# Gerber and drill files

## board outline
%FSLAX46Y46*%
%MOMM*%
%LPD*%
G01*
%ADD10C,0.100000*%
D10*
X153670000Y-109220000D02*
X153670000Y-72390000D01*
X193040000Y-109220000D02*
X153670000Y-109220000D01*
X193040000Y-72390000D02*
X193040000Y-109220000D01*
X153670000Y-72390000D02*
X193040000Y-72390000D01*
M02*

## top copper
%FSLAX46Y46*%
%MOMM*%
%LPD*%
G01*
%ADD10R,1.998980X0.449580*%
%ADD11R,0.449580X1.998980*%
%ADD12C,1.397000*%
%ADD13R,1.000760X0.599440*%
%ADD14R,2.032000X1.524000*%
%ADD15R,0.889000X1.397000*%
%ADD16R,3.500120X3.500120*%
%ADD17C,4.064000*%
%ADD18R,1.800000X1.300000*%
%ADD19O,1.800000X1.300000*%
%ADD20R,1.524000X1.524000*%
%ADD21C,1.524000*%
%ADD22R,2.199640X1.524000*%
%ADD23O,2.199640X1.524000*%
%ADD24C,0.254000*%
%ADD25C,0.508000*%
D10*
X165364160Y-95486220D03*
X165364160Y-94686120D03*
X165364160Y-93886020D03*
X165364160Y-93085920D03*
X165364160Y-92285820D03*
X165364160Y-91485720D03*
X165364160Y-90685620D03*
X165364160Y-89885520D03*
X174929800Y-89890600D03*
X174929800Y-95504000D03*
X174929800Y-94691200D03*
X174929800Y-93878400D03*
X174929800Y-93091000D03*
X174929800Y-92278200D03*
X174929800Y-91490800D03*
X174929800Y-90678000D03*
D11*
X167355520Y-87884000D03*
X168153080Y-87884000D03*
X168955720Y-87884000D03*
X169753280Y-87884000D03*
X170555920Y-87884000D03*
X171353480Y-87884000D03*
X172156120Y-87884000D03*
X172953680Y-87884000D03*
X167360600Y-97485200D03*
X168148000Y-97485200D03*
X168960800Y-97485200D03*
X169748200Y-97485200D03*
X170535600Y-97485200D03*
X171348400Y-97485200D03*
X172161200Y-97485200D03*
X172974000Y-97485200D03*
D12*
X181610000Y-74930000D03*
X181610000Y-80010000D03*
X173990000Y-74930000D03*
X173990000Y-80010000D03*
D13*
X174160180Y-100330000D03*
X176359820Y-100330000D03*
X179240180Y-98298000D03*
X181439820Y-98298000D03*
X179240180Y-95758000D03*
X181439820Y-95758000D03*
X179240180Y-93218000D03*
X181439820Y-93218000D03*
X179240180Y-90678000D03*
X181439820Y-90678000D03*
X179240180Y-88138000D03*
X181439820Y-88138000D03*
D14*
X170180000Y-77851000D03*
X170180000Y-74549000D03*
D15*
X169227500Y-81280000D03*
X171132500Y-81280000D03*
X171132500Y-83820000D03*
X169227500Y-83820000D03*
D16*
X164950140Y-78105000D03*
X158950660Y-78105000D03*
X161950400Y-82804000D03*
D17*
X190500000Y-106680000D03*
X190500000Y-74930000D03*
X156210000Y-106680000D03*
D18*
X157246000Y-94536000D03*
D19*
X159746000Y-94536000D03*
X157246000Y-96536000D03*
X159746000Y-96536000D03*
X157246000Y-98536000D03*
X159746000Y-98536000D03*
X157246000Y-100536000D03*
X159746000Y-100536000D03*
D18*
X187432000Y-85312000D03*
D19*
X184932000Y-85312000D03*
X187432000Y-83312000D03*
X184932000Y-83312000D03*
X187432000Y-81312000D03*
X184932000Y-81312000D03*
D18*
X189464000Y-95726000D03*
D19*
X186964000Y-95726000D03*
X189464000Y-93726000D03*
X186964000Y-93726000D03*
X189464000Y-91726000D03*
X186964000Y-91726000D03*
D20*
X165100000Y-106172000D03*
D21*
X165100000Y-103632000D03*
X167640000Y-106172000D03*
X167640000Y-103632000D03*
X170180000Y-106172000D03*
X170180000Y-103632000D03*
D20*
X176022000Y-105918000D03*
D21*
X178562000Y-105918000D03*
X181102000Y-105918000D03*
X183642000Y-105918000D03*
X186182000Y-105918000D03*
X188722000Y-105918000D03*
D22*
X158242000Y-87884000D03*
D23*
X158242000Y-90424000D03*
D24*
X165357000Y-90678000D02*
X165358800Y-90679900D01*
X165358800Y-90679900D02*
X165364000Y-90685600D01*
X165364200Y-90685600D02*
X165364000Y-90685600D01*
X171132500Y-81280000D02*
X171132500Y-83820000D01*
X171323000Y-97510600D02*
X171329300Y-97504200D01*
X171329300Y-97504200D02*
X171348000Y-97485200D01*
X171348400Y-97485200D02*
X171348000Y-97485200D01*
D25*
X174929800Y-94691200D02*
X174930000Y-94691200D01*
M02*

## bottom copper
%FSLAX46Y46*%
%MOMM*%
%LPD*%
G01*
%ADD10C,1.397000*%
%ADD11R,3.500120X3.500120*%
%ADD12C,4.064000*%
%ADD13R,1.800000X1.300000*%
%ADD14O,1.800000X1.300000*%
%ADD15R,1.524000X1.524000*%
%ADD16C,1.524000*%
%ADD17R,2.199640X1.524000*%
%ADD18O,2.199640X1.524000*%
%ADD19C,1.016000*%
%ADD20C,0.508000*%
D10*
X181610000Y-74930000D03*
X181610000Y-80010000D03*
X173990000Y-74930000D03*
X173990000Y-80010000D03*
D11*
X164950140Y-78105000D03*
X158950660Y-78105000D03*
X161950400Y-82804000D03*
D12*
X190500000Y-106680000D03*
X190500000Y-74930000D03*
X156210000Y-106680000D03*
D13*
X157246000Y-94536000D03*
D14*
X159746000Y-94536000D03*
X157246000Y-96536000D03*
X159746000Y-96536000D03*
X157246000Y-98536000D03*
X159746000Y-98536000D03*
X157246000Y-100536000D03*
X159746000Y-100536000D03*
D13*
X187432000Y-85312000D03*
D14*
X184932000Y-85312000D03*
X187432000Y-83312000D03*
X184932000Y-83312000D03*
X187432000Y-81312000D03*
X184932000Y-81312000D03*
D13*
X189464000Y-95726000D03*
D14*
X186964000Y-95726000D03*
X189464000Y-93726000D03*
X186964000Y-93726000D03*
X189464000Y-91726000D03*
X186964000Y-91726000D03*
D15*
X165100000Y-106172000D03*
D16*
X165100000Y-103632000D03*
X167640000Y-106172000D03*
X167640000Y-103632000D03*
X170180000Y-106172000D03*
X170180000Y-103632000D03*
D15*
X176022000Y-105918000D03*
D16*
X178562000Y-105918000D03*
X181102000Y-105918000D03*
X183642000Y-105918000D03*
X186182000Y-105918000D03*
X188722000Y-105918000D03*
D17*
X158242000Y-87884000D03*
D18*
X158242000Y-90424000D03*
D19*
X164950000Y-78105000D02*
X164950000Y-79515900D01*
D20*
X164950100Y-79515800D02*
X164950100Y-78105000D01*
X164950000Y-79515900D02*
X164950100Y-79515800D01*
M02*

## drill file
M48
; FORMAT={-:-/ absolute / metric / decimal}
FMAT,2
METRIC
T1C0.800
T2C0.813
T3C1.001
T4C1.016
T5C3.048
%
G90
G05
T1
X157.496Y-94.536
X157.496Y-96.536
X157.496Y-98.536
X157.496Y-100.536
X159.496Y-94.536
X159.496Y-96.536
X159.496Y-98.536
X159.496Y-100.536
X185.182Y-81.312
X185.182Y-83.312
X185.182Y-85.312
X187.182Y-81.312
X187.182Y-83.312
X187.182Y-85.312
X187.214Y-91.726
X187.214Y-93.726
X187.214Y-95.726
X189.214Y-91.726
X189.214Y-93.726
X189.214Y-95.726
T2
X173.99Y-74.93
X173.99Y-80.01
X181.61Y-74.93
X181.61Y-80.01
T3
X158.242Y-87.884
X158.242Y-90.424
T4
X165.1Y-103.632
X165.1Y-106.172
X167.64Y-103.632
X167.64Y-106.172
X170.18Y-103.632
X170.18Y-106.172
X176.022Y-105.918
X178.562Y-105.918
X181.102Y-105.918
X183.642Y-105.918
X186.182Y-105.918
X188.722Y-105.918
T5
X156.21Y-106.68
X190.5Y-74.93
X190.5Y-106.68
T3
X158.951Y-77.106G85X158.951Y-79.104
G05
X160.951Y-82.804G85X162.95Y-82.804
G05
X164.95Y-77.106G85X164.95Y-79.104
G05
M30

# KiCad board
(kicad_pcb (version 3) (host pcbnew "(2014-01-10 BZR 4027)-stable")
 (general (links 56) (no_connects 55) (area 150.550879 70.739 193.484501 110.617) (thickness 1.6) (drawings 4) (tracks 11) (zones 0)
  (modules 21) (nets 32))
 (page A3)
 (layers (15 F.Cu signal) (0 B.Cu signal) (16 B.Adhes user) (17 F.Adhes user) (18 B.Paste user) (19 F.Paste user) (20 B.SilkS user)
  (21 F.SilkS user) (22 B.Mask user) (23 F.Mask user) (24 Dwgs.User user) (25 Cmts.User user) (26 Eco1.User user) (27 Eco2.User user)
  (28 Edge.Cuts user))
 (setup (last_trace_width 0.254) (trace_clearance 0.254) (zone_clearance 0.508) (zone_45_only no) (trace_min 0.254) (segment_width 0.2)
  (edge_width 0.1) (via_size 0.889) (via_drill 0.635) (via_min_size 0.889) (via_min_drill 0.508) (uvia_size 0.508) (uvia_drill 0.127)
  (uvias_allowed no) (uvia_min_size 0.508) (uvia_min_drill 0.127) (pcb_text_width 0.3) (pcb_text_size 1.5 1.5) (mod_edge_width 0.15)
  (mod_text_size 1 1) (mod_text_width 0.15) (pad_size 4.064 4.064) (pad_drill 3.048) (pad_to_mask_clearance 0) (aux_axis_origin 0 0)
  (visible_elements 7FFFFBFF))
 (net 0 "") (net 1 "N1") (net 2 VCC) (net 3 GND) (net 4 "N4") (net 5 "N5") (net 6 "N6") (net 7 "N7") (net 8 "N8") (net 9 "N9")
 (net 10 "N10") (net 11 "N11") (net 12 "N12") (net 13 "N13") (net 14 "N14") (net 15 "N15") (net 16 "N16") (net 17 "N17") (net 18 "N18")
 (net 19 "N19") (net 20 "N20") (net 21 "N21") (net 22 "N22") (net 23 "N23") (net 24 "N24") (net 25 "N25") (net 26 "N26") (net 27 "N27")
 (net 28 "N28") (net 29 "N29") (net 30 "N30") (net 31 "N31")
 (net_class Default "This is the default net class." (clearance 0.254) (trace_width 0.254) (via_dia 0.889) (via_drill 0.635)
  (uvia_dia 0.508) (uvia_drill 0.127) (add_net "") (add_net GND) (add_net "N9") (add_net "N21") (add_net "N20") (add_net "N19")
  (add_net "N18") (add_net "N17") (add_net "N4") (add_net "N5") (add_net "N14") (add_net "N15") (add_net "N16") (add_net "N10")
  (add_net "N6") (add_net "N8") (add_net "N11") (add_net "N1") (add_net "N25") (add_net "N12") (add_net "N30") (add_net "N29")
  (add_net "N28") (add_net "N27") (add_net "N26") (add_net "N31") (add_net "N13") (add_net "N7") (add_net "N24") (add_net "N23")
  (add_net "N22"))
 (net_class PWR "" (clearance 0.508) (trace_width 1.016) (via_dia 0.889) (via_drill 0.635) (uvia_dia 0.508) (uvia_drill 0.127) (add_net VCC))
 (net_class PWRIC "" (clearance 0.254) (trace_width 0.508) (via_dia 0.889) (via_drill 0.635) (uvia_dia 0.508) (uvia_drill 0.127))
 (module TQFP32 (layer F.Cu) (at 170.18 92.71)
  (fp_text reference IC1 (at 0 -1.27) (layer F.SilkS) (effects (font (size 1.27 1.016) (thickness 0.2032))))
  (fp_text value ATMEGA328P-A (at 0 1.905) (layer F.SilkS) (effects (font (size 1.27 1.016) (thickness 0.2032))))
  (pad 8 smd rect (at -4.81584 2.77622) (size 1.99898 0.44958) (layers F.Cu F.Paste F.Mask) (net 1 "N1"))
  (pad 7 smd rect (at -4.81584 1.97612) (size 1.99898 0.44958) (layers F.Cu F.Paste F.Mask))
  (pad 6 smd rect (at -4.81584 1.17602) (size 1.99898 0.44958) (layers F.Cu F.Paste F.Mask) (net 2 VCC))
  (pad 5 smd rect (at -4.81584 0.37592) (size 1.99898 0.44958) (layers F.Cu F.Paste F.Mask) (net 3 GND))
  (pad 4 smd rect (at -4.81584 -0.42418) (size 1.99898 0.44958) (layers F.Cu F.Paste F.Mask) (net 2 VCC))
  (pad 3 smd rect (at -4.81584 -1.22428) (size 1.99898 0.44958) (layers F.Cu F.Paste F.Mask) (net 3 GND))
  (pad 2 smd rect (at -4.81584 -2.02438) (size 1.99898 0.44958) (layers F.Cu F.Paste F.Mask) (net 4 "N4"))
  (pad 1 smd rect (at -4.81584 -2.82448) (size 1.99898 0.44958) (layers F.Cu F.Paste F.Mask) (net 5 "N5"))
  (pad 24 smd rect (at 4.7498 -2.8194) (size 1.99898 0.44958) (layers F.Cu F.Paste F.Mask) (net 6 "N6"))
  (pad 17 smd rect (at 4.7498 2.794) (size 1.99898 0.44958) (layers F.Cu F.Paste F.Mask) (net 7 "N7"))
  (pad 18 smd rect (at 4.7498 1.9812) (size 1.99898 0.44958) (layers F.Cu F.Paste F.Mask) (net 2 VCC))
  (pad 19 smd rect (at 4.7498 1.1684) (size 1.99898 0.44958) (layers F.Cu F.Paste F.Mask))
  (pad 20 smd rect (at 4.7498 0.381) (size 1.99898 0.44958) (layers F.Cu F.Paste F.Mask))
  (pad 21 smd rect (at 4.7498 -0.4318) (size 1.99898 0.44958) (layers F.Cu F.Paste F.Mask) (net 3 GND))
  (pad 22 smd rect (at 4.7498 -1.2192) (size 1.99898 0.44958) (layers F.Cu F.Paste F.Mask))
  (pad 23 smd rect (at 4.7498 -2.032) (size 1.99898 0.44958) (layers F.Cu F.Paste F.Mask) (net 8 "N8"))
  (pad 32 smd rect (at -2.82448 -4.826) (size 0.44958 1.99898) (layers F.Cu F.Paste F.Mask) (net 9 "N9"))
  (pad 31 smd rect (at -2.02692 -4.826) (size 0.44958 1.99898) (layers F.Cu F.Paste F.Mask) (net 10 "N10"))
  (pad 30 smd rect (at -1.22428 -4.826) (size 0.44958 1.99898) (layers F.Cu F.Paste F.Mask) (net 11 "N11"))
  (pad 29 smd rect (at -0.42672 -4.826) (size 0.44958 1.99898) (layers F.Cu F.Paste F.Mask) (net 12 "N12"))
  (pad 28 smd rect (at 0.37592 -4.826) (size 0.44958 1.99898) (layers F.Cu F.Paste F.Mask) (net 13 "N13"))
  (pad 27 smd rect (at 1.17348 -4.826) (size 0.44958 1.99898) (layers F.Cu F.Paste F.Mask) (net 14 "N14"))
  (pad 26 smd rect (at 1.97612 -4.826) (size 0.44958 1.99898) (layers F.Cu F.Paste F.Mask) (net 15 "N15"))
  (pad 25 smd rect (at 2.77368 -4.826) (size 0.44958 1.99898) (layers F.Cu F.Paste F.Mask) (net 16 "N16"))
  (pad 9 smd rect (at -2.8194 4.7752) (size 0.44958 1.99898) (layers F.Cu F.Paste F.Mask) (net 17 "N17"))
  (pad 10 smd rect (at -2.032 4.7752) (size 0.44958 1.99898) (layers F.Cu F.Paste F.Mask) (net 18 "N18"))
  (pad 11 smd rect (at -1.2192 4.7752) (size 0.44958 1.99898) (layers F.Cu F.Paste F.Mask) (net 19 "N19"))
  (pad 12 smd rect (at -0.4318 4.7752) (size 0.44958 1.99898) (layers F.Cu F.Paste F.Mask) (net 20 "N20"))
  (pad 13 smd rect (at 0.3556 4.7752) (size 0.44958 1.99898) (layers F.Cu F.Paste F.Mask) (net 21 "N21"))
  (pad 14 smd rect (at 1.1684 4.7752) (size 0.44958 1.99898) (layers F.Cu F.Paste F.Mask) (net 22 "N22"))
  (pad 15 smd rect (at 1.9812 4.7752) (size 0.44958 1.99898) (layers F.Cu F.Paste F.Mask) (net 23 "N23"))
  (pad 16 smd rect (at 2.794 4.7752) (size 0.44958 1.99898) (layers F.Cu F.Paste F.Mask) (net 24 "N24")))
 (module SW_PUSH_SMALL (layer F.Cu) (at 177.8 77.47)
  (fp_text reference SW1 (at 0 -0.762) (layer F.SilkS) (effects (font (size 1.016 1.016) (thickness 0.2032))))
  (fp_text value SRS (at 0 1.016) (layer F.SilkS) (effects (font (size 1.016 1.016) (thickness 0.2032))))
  (pad 1 thru_hole circle (at 3.81 -2.54) (size 1.397 1.397) (drill 0.8128) (layers *.Cu *.Mask F.SilkS) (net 1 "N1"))
  (pad 2 thru_hole circle (at 3.81 2.54) (size 1.397 1.397) (drill 0.8128) (layers *.Cu *.Mask F.SilkS) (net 3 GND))
  (pad 1 thru_hole circle (at -3.81 -2.54) (size 1.397 1.397) (drill 0.8128) (layers *.Cu *.Mask F.SilkS) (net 1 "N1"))
  (pad 2 thru_hole circle (at -3.81 2.54) (size 1.397 1.397) (drill 0.8128) (layers *.Cu *.Mask F.SilkS) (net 3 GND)))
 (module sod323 (layer F.Cu) (at 175.26 100.33 180)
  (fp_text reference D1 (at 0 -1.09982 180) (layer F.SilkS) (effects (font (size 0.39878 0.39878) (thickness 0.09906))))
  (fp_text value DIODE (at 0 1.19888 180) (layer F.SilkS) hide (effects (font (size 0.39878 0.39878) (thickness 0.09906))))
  (pad 2 smd rect (at 1.09982 0 180) (size 1.00076 0.59944) (layers F.Cu F.Paste F.Mask) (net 20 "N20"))
  (pad 1 smd rect (at -1.09982 0 180) (size 1.00076 0.59944) (layers F.Cu F.Paste F.Mask) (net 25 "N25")))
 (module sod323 (layer F.Cu) (at 180.34 98.298 180)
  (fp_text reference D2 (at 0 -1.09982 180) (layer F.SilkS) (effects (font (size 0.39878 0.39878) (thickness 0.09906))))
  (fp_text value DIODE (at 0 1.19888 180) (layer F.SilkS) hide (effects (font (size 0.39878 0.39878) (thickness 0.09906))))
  (pad 2 smd rect (at 1.09982 0 180) (size 1.00076 0.59944) (layers F.Cu F.Paste F.Mask) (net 21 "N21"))
  (pad 1 smd rect (at -1.09982 0 180) (size 1.00076 0.59944) (layers F.Cu F.Paste F.Mask) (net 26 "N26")))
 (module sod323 (layer F.Cu) (at 180.34 95.758 180)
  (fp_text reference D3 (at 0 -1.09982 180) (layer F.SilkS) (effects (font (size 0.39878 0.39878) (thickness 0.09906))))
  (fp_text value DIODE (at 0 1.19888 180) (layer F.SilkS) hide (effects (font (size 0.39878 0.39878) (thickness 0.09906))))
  (pad 2 smd rect (at 1.09982 0 180) (size 1.00076 0.59944) (layers F.Cu F.Paste F.Mask) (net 22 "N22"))
  (pad 1 smd rect (at -1.09982 0 180) (size 1.00076 0.59944) (layers F.Cu F.Paste F.Mask) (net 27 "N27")))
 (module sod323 (layer F.Cu) (at 180.34 93.218 180)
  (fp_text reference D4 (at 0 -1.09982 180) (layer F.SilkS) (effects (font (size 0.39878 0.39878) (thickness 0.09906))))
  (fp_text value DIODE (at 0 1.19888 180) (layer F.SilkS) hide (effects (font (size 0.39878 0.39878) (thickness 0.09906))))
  (pad 2 smd rect (at 1.09982 0 180) (size 1.00076 0.59944) (layers F.Cu F.Paste F.Mask) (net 23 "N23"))
  (pad 1 smd rect (at -1.09982 0 180) (size 1.00076 0.59944) (layers F.Cu F.Paste F.Mask) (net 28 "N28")))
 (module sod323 (layer F.Cu) (at 180.34 90.678 180)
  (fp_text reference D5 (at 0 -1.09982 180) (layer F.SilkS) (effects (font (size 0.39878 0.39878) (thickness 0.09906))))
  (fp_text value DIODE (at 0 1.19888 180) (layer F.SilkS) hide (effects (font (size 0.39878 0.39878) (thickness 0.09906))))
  (pad 2 smd rect (at 1.09982 0 180) (size 1.00076 0.59944) (layers F.Cu F.Paste F.Mask) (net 24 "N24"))
  (pad 1 smd rect (at -1.09982 0 180) (size 1.00076 0.59944) (layers F.Cu F.Paste F.Mask) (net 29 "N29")))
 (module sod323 (layer F.Cu) (at 180.34 88.138 180)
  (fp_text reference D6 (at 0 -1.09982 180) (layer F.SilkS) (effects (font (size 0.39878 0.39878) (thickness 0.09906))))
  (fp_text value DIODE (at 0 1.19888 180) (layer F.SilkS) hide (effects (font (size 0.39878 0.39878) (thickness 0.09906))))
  (pad 2 smd rect (at 1.09982 0 180) (size 1.00076 0.59944) (layers F.Cu F.Paste F.Mask) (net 7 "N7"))
  (pad 1 smd rect (at -1.09982 0 180) (size 1.00076 0.59944) (layers F.Cu F.Paste F.Mask) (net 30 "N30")))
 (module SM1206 (layer F.Cu) (at 170.18 76.2 90)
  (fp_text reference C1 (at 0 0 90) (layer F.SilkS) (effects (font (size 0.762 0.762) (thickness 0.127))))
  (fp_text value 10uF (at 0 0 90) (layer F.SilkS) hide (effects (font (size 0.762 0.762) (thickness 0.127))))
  (pad 1 smd rect (at -1.651 0 90) (size 1.524 2.032) (layers F.Cu F.Paste F.Mask) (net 2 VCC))
  (pad 2 smd rect (at 1.651 0 90) (size 1.524 2.032) (layers F.Cu F.Paste F.Mask) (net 3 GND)))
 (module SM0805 (layer F.Cu) (at 170.18 81.28)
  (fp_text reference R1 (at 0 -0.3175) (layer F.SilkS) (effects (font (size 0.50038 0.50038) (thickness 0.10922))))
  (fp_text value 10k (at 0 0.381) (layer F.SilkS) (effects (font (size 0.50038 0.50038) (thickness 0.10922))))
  (pad 1 smd rect (at -0.9525 0) (size 0.889 1.397) (layers F.Cu F.Paste F.Mask) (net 2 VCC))
  (pad 2 smd rect (at 0.9525 0) (size 0.889 1.397) (layers F.Cu F.Paste F.Mask) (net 12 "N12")))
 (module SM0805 (layer F.Cu) (at 170.18 83.82 180)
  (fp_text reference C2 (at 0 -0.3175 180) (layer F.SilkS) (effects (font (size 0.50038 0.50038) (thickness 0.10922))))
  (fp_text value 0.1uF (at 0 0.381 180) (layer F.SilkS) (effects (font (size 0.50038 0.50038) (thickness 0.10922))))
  (pad 1 smd rect (at -0.9525 0 180) (size 0.889 1.397) (layers F.Cu F.Paste F.Mask) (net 12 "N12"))
  (pad 2 smd rect (at 0.9525 0 180) (size 0.889 1.397) (layers F.Cu F.Paste F.Mask) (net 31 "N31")))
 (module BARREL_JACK (layer F.Cu) (at 158.75 78.105)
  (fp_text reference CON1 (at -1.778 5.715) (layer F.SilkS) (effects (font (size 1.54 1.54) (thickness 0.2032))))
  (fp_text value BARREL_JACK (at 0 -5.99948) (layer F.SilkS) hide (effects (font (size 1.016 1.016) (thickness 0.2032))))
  (pad 1 thru_hole rect (at 6.20014 0) (size 3.50012 3.50012) (drill oval 1.00076 2.99974) (layers *.Cu *.Mask F.SilkS) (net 2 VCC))
  (pad 2 thru_hole rect (at 0.20066 0) (size 3.50012 3.50012) (drill oval 1.00076 2.99974) (layers *.Cu *.Mask F.SilkS) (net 3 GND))
  (pad 3 thru_hole rect (at 3.2004 4.699) (size 3.50012 3.50012) (drill oval 2.99974 1.00076) (layers *.Cu *.Mask F.SilkS) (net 3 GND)))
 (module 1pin (layer F.Cu) (at 190.5 106.68)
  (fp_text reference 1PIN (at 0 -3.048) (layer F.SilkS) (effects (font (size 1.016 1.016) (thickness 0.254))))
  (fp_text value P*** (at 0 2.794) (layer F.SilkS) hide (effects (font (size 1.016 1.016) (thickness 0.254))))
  (pad 1 thru_hole circle (at 0 0) (size 4.064 4.064) (drill 3.048) (layers *.Cu *.Mask F.SilkS)))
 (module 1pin (layer F.Cu) (at 190.5 74.93)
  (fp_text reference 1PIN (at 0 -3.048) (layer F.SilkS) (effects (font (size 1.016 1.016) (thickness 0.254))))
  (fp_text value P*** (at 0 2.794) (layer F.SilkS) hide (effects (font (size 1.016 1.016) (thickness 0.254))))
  (pad 1 thru_hole circle (at 0 0) (size 4.064 4.064) (drill 3.048) (layers *.Cu *.Mask F.SilkS)))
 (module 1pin (layer F.Cu) (at 156.21 106.68)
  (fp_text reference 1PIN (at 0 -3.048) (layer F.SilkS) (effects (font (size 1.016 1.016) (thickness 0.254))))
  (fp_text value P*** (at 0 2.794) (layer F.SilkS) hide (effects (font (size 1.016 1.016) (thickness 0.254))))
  (pad 1 thru_hole circle (at 0 0) (size 4.064 4.064) (drill 3.048) (layers *.Cu *.Mask F.SilkS) (clearance 1)))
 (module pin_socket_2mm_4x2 (layer F.Cu) (at 158.496 97.536 270)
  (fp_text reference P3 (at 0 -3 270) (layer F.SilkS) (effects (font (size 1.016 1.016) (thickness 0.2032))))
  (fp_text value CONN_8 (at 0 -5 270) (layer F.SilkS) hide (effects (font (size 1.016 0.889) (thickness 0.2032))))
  (pad 1 thru_hole rect (at -3 1 270) (size 1.3 1.8) (drill 0.8 (offset 0 0.25)) (layers *.Cu *.Mask F.SilkS) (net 11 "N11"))
  (pad 2 thru_hole oval (at -3 -1 270) (size 1.3 1.8) (drill 0.8 (offset 0 -0.25)) (layers *.Cu *.Mask F.SilkS) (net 10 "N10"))
  (pad 3 thru_hole oval (at -1 1 270) (size 1.3 1.8) (drill 0.8 (offset 0 0.25)) (layers *.Cu *.Mask F.SilkS) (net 9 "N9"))
  (pad 4 thru_hole oval (at -1 -1 270) (size 1.3 1.8) (drill 0.8 (offset 0 -0.25)) (layers *.Cu *.Mask F.SilkS) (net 5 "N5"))
  (pad 5 thru_hole oval (at 1 1 270) (size 1.3 1.8) (drill 0.8 (offset 0 0.25)) (layers *.Cu *.Mask F.SilkS) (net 4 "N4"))
  (pad 6 thru_hole oval (at 1 -1 270) (size 1.3 1.8) (drill 0.8 (offset 0 -0.25)) (layers *.Cu *.Mask F.SilkS) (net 17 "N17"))
  (pad 7 thru_hole oval (at 3 1 270) (size 1.3 1.8) (drill 0.8 (offset 0 0.25)) (layers *.Cu *.Mask F.SilkS) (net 18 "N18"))
  (pad 8 thru_hole oval (at 3 -1 270) (size 1.3 1.8) (drill 0.8 (offset 0 -0.25)) (layers *.Cu *.Mask F.SilkS) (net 19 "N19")))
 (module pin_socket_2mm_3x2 (layer F.Cu) (at 186.182 83.312 90)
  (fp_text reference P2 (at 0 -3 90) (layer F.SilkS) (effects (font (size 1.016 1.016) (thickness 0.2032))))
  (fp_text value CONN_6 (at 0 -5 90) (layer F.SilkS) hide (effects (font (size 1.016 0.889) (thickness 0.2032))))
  (pad 1 thru_hole rect (at -2 1 90) (size 1.3 1.8) (drill 0.8 (offset 0 0.25)) (layers *.Cu *.Mask F.SilkS) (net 8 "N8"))
  (pad 2 thru_hole oval (at -2 -1 90) (size 1.3 1.8) (drill 0.8 (offset 0 -0.25)) (layers *.Cu *.Mask F.SilkS) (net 6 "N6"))
  (pad 3 thru_hole oval (at 0 1 90) (size 1.3 1.8) (drill 0.8 (offset 0 0.25)) (layers *.Cu *.Mask F.SilkS) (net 16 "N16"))
  (pad 4 thru_hole oval (at 0 -1 90) (size 1.3 1.8) (drill 0.8 (offset 0 -0.25)) (layers *.Cu *.Mask F.SilkS) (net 15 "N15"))
  (pad 5 thru_hole oval (at 2 1 90) (size 1.3 1.8) (drill 0.8 (offset 0 0.25)) (layers *.Cu *.Mask F.SilkS) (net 14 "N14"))
  (pad 6 thru_hole oval (at 2 -1 90) (size 1.3 1.8) (drill 0.8 (offset 0 -0.25)) (layers *.Cu *.Mask F.SilkS) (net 13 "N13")))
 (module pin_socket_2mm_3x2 (layer F.Cu) (at 188.214 93.726 90)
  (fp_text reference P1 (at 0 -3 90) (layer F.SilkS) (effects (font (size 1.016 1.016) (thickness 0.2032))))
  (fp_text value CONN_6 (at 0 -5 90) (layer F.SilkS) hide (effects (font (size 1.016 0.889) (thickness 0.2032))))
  (pad 1 thru_hole rect (at -2 1 90) (size 1.3 1.8) (drill 0.8 (offset 0 0.25)) (layers *.Cu *.Mask F.SilkS) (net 25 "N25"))
  (pad 2 thru_hole oval (at -2 -1 90) (size 1.3 1.8) (drill 0.8 (offset 0 -0.25)) (layers *.Cu *.Mask F.SilkS) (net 26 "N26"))
  (pad 3 thru_hole oval (at 0 1 90) (size 1.3 1.8) (drill 0.8 (offset 0 0.25)) (layers *.Cu *.Mask F.SilkS) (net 27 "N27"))
  (pad 4 thru_hole oval (at 0 -1 90) (size 1.3 1.8) (drill 0.8 (offset 0 -0.25)) (layers *.Cu *.Mask F.SilkS) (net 28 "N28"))
  (pad 5 thru_hole oval (at 2 1 90) (size 1.3 1.8) (drill 0.8 (offset 0 0.25)) (layers *.Cu *.Mask F.SilkS) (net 29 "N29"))
  (pad 6 thru_hole oval (at 2 -1 90) (size 1.3 1.8) (drill 0.8 (offset 0 -0.25)) (layers *.Cu *.Mask F.SilkS) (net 30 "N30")))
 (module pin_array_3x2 (layer F.Cu) (at 167.64 104.902)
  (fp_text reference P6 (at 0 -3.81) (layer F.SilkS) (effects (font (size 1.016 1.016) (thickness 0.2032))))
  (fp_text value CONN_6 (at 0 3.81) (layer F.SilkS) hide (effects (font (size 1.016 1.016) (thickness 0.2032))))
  (pad 1 thru_hole rect (at -2.54 1.27) (size 1.524 1.524) (drill 1.016) (layers *.Cu *.Mask F.SilkS) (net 24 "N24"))
  (pad 2 thru_hole circle (at -2.54 -1.27) (size 1.524 1.524) (drill 1.016) (layers *.Cu *.Mask F.SilkS) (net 2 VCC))
  (pad 3 thru_hole circle (at 0 1.27) (size 1.524 1.524) (drill 1.016) (layers *.Cu *.Mask F.SilkS) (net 7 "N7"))
  (pad 4 thru_hole circle (at 0 -1.27) (size 1.524 1.524) (drill 1.016) (layers *.Cu *.Mask F.SilkS) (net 23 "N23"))
  (pad 5 thru_hole circle (at 2.54 1.27) (size 1.524 1.524) (drill 1.016) (layers *.Cu *.Mask F.SilkS) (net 12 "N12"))
  (pad 6 thru_hole circle (at 2.54 -1.27) (size 1.524 1.524) (drill 1.016) (layers *.Cu *.Mask F.SilkS) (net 3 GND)))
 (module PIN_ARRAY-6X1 (layer F.Cu) (at 182.372 105.918)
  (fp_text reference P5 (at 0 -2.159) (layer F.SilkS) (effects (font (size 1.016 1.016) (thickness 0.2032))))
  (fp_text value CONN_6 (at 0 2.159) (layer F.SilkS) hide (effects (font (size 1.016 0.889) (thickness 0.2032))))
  (pad 1 thru_hole rect (at -6.35 0) (size 1.524 1.524) (drill 1.016) (layers *.Cu *.Mask F.SilkS) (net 31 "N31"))
  (pad 2 thru_hole circle (at -3.81 0) (size 1.524 1.524) (drill 1.016) (layers *.Cu *.Mask F.SilkS) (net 10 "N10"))
  (pad 3 thru_hole circle (at -1.27 0) (size 1.524 1.524) (drill 1.016) (layers *.Cu *.Mask F.SilkS) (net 11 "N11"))
  (pad 4 thru_hole circle (at 1.27 0) (size 1.524 1.524) (drill 1.016) (layers *.Cu *.Mask F.SilkS) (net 2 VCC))
  (pad 5 thru_hole circle (at 3.81 0) (size 1.524 1.524) (drill 1.016) (layers *.Cu *.Mask F.SilkS) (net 3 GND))
  (pad 6 thru_hole circle (at 6.35 0) (size 1.524 1.524) (drill 1.016) (layers *.Cu *.Mask F.SilkS) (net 3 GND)))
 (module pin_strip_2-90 (layer F.Cu) (at 158.242 89.154 270)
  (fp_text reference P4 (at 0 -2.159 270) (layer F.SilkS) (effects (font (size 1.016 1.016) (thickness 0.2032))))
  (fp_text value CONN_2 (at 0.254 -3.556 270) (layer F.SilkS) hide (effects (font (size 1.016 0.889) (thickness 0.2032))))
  (pad 1 thru_hole rect (at -1.27 0 270) (size 1.524 2.19964) (drill 1.00076) (layers *.Cu *.Mask F.SilkS) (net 2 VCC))
  (pad 2 thru_hole oval (at 1.27 0 270) (size 1.524 2.19964) (drill 1.00076) (layers *.Cu *.Mask F.SilkS) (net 3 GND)))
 (gr_line (start 153.67 109.22) (end 153.67 72.39) (angle 90) (layer Edge.Cuts) (width 0.1))
 (gr_line (start 193.04 109.22) (end 153.67 109.22) (angle 90) (layer Edge.Cuts) (width 0.1))
 (gr_line (start 193.04 72.39) (end 193.04 109.22) (angle 90) (layer Edge.Cuts) (width 0.1))
 (gr_line (start 153.67 72.39) (end 193.04 72.39) (angle 90) (layer Edge.Cuts) (width 0.1))
 (segment (start 165.357 90.678) (end 165.3588 90.6799) (width 0.254) (layer F.Cu) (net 4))
 (segment (start 165.3588 90.6799) (end 165.364 90.6856) (width 0.254) (layer F.Cu) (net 4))
 (segment (start 165.3642 90.6856) (end 165.364 90.6856) (width 0.254) (layer F.Cu) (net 4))
 (segment (start 171.1325 81.28) (end 171.1325 83.82) (width 0.254) (layer F.Cu) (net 12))
 (segment (start 171.323 97.5106) (end 171.3293 97.5042) (width 0.254) (layer F.Cu) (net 22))
 (segment (start 171.3293 97.5042) (end 171.348 97.4852) (width 0.254) (layer F.Cu) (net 22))
 (segment (start 171.3484 97.4852) (end 171.348 97.4852) (width 0.254) (layer F.Cu) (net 22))
 (segment (start 174.9298 94.6912) (end 174.93 94.6912) (width 0.508) (layer F.Cu) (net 2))
 (segment (start 164.95 78.105) (end 164.95 79.5159) (width 1.016) (layer B.Cu) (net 2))
 (segment (start 164.9501 79.5158) (end 164.9501 78.105) (width 0.508) (layer B.Cu) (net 2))
 (segment (start 164.95 79.5159) (end 164.9501 79.5158) (width 0.508) (layer B.Cu) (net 2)))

